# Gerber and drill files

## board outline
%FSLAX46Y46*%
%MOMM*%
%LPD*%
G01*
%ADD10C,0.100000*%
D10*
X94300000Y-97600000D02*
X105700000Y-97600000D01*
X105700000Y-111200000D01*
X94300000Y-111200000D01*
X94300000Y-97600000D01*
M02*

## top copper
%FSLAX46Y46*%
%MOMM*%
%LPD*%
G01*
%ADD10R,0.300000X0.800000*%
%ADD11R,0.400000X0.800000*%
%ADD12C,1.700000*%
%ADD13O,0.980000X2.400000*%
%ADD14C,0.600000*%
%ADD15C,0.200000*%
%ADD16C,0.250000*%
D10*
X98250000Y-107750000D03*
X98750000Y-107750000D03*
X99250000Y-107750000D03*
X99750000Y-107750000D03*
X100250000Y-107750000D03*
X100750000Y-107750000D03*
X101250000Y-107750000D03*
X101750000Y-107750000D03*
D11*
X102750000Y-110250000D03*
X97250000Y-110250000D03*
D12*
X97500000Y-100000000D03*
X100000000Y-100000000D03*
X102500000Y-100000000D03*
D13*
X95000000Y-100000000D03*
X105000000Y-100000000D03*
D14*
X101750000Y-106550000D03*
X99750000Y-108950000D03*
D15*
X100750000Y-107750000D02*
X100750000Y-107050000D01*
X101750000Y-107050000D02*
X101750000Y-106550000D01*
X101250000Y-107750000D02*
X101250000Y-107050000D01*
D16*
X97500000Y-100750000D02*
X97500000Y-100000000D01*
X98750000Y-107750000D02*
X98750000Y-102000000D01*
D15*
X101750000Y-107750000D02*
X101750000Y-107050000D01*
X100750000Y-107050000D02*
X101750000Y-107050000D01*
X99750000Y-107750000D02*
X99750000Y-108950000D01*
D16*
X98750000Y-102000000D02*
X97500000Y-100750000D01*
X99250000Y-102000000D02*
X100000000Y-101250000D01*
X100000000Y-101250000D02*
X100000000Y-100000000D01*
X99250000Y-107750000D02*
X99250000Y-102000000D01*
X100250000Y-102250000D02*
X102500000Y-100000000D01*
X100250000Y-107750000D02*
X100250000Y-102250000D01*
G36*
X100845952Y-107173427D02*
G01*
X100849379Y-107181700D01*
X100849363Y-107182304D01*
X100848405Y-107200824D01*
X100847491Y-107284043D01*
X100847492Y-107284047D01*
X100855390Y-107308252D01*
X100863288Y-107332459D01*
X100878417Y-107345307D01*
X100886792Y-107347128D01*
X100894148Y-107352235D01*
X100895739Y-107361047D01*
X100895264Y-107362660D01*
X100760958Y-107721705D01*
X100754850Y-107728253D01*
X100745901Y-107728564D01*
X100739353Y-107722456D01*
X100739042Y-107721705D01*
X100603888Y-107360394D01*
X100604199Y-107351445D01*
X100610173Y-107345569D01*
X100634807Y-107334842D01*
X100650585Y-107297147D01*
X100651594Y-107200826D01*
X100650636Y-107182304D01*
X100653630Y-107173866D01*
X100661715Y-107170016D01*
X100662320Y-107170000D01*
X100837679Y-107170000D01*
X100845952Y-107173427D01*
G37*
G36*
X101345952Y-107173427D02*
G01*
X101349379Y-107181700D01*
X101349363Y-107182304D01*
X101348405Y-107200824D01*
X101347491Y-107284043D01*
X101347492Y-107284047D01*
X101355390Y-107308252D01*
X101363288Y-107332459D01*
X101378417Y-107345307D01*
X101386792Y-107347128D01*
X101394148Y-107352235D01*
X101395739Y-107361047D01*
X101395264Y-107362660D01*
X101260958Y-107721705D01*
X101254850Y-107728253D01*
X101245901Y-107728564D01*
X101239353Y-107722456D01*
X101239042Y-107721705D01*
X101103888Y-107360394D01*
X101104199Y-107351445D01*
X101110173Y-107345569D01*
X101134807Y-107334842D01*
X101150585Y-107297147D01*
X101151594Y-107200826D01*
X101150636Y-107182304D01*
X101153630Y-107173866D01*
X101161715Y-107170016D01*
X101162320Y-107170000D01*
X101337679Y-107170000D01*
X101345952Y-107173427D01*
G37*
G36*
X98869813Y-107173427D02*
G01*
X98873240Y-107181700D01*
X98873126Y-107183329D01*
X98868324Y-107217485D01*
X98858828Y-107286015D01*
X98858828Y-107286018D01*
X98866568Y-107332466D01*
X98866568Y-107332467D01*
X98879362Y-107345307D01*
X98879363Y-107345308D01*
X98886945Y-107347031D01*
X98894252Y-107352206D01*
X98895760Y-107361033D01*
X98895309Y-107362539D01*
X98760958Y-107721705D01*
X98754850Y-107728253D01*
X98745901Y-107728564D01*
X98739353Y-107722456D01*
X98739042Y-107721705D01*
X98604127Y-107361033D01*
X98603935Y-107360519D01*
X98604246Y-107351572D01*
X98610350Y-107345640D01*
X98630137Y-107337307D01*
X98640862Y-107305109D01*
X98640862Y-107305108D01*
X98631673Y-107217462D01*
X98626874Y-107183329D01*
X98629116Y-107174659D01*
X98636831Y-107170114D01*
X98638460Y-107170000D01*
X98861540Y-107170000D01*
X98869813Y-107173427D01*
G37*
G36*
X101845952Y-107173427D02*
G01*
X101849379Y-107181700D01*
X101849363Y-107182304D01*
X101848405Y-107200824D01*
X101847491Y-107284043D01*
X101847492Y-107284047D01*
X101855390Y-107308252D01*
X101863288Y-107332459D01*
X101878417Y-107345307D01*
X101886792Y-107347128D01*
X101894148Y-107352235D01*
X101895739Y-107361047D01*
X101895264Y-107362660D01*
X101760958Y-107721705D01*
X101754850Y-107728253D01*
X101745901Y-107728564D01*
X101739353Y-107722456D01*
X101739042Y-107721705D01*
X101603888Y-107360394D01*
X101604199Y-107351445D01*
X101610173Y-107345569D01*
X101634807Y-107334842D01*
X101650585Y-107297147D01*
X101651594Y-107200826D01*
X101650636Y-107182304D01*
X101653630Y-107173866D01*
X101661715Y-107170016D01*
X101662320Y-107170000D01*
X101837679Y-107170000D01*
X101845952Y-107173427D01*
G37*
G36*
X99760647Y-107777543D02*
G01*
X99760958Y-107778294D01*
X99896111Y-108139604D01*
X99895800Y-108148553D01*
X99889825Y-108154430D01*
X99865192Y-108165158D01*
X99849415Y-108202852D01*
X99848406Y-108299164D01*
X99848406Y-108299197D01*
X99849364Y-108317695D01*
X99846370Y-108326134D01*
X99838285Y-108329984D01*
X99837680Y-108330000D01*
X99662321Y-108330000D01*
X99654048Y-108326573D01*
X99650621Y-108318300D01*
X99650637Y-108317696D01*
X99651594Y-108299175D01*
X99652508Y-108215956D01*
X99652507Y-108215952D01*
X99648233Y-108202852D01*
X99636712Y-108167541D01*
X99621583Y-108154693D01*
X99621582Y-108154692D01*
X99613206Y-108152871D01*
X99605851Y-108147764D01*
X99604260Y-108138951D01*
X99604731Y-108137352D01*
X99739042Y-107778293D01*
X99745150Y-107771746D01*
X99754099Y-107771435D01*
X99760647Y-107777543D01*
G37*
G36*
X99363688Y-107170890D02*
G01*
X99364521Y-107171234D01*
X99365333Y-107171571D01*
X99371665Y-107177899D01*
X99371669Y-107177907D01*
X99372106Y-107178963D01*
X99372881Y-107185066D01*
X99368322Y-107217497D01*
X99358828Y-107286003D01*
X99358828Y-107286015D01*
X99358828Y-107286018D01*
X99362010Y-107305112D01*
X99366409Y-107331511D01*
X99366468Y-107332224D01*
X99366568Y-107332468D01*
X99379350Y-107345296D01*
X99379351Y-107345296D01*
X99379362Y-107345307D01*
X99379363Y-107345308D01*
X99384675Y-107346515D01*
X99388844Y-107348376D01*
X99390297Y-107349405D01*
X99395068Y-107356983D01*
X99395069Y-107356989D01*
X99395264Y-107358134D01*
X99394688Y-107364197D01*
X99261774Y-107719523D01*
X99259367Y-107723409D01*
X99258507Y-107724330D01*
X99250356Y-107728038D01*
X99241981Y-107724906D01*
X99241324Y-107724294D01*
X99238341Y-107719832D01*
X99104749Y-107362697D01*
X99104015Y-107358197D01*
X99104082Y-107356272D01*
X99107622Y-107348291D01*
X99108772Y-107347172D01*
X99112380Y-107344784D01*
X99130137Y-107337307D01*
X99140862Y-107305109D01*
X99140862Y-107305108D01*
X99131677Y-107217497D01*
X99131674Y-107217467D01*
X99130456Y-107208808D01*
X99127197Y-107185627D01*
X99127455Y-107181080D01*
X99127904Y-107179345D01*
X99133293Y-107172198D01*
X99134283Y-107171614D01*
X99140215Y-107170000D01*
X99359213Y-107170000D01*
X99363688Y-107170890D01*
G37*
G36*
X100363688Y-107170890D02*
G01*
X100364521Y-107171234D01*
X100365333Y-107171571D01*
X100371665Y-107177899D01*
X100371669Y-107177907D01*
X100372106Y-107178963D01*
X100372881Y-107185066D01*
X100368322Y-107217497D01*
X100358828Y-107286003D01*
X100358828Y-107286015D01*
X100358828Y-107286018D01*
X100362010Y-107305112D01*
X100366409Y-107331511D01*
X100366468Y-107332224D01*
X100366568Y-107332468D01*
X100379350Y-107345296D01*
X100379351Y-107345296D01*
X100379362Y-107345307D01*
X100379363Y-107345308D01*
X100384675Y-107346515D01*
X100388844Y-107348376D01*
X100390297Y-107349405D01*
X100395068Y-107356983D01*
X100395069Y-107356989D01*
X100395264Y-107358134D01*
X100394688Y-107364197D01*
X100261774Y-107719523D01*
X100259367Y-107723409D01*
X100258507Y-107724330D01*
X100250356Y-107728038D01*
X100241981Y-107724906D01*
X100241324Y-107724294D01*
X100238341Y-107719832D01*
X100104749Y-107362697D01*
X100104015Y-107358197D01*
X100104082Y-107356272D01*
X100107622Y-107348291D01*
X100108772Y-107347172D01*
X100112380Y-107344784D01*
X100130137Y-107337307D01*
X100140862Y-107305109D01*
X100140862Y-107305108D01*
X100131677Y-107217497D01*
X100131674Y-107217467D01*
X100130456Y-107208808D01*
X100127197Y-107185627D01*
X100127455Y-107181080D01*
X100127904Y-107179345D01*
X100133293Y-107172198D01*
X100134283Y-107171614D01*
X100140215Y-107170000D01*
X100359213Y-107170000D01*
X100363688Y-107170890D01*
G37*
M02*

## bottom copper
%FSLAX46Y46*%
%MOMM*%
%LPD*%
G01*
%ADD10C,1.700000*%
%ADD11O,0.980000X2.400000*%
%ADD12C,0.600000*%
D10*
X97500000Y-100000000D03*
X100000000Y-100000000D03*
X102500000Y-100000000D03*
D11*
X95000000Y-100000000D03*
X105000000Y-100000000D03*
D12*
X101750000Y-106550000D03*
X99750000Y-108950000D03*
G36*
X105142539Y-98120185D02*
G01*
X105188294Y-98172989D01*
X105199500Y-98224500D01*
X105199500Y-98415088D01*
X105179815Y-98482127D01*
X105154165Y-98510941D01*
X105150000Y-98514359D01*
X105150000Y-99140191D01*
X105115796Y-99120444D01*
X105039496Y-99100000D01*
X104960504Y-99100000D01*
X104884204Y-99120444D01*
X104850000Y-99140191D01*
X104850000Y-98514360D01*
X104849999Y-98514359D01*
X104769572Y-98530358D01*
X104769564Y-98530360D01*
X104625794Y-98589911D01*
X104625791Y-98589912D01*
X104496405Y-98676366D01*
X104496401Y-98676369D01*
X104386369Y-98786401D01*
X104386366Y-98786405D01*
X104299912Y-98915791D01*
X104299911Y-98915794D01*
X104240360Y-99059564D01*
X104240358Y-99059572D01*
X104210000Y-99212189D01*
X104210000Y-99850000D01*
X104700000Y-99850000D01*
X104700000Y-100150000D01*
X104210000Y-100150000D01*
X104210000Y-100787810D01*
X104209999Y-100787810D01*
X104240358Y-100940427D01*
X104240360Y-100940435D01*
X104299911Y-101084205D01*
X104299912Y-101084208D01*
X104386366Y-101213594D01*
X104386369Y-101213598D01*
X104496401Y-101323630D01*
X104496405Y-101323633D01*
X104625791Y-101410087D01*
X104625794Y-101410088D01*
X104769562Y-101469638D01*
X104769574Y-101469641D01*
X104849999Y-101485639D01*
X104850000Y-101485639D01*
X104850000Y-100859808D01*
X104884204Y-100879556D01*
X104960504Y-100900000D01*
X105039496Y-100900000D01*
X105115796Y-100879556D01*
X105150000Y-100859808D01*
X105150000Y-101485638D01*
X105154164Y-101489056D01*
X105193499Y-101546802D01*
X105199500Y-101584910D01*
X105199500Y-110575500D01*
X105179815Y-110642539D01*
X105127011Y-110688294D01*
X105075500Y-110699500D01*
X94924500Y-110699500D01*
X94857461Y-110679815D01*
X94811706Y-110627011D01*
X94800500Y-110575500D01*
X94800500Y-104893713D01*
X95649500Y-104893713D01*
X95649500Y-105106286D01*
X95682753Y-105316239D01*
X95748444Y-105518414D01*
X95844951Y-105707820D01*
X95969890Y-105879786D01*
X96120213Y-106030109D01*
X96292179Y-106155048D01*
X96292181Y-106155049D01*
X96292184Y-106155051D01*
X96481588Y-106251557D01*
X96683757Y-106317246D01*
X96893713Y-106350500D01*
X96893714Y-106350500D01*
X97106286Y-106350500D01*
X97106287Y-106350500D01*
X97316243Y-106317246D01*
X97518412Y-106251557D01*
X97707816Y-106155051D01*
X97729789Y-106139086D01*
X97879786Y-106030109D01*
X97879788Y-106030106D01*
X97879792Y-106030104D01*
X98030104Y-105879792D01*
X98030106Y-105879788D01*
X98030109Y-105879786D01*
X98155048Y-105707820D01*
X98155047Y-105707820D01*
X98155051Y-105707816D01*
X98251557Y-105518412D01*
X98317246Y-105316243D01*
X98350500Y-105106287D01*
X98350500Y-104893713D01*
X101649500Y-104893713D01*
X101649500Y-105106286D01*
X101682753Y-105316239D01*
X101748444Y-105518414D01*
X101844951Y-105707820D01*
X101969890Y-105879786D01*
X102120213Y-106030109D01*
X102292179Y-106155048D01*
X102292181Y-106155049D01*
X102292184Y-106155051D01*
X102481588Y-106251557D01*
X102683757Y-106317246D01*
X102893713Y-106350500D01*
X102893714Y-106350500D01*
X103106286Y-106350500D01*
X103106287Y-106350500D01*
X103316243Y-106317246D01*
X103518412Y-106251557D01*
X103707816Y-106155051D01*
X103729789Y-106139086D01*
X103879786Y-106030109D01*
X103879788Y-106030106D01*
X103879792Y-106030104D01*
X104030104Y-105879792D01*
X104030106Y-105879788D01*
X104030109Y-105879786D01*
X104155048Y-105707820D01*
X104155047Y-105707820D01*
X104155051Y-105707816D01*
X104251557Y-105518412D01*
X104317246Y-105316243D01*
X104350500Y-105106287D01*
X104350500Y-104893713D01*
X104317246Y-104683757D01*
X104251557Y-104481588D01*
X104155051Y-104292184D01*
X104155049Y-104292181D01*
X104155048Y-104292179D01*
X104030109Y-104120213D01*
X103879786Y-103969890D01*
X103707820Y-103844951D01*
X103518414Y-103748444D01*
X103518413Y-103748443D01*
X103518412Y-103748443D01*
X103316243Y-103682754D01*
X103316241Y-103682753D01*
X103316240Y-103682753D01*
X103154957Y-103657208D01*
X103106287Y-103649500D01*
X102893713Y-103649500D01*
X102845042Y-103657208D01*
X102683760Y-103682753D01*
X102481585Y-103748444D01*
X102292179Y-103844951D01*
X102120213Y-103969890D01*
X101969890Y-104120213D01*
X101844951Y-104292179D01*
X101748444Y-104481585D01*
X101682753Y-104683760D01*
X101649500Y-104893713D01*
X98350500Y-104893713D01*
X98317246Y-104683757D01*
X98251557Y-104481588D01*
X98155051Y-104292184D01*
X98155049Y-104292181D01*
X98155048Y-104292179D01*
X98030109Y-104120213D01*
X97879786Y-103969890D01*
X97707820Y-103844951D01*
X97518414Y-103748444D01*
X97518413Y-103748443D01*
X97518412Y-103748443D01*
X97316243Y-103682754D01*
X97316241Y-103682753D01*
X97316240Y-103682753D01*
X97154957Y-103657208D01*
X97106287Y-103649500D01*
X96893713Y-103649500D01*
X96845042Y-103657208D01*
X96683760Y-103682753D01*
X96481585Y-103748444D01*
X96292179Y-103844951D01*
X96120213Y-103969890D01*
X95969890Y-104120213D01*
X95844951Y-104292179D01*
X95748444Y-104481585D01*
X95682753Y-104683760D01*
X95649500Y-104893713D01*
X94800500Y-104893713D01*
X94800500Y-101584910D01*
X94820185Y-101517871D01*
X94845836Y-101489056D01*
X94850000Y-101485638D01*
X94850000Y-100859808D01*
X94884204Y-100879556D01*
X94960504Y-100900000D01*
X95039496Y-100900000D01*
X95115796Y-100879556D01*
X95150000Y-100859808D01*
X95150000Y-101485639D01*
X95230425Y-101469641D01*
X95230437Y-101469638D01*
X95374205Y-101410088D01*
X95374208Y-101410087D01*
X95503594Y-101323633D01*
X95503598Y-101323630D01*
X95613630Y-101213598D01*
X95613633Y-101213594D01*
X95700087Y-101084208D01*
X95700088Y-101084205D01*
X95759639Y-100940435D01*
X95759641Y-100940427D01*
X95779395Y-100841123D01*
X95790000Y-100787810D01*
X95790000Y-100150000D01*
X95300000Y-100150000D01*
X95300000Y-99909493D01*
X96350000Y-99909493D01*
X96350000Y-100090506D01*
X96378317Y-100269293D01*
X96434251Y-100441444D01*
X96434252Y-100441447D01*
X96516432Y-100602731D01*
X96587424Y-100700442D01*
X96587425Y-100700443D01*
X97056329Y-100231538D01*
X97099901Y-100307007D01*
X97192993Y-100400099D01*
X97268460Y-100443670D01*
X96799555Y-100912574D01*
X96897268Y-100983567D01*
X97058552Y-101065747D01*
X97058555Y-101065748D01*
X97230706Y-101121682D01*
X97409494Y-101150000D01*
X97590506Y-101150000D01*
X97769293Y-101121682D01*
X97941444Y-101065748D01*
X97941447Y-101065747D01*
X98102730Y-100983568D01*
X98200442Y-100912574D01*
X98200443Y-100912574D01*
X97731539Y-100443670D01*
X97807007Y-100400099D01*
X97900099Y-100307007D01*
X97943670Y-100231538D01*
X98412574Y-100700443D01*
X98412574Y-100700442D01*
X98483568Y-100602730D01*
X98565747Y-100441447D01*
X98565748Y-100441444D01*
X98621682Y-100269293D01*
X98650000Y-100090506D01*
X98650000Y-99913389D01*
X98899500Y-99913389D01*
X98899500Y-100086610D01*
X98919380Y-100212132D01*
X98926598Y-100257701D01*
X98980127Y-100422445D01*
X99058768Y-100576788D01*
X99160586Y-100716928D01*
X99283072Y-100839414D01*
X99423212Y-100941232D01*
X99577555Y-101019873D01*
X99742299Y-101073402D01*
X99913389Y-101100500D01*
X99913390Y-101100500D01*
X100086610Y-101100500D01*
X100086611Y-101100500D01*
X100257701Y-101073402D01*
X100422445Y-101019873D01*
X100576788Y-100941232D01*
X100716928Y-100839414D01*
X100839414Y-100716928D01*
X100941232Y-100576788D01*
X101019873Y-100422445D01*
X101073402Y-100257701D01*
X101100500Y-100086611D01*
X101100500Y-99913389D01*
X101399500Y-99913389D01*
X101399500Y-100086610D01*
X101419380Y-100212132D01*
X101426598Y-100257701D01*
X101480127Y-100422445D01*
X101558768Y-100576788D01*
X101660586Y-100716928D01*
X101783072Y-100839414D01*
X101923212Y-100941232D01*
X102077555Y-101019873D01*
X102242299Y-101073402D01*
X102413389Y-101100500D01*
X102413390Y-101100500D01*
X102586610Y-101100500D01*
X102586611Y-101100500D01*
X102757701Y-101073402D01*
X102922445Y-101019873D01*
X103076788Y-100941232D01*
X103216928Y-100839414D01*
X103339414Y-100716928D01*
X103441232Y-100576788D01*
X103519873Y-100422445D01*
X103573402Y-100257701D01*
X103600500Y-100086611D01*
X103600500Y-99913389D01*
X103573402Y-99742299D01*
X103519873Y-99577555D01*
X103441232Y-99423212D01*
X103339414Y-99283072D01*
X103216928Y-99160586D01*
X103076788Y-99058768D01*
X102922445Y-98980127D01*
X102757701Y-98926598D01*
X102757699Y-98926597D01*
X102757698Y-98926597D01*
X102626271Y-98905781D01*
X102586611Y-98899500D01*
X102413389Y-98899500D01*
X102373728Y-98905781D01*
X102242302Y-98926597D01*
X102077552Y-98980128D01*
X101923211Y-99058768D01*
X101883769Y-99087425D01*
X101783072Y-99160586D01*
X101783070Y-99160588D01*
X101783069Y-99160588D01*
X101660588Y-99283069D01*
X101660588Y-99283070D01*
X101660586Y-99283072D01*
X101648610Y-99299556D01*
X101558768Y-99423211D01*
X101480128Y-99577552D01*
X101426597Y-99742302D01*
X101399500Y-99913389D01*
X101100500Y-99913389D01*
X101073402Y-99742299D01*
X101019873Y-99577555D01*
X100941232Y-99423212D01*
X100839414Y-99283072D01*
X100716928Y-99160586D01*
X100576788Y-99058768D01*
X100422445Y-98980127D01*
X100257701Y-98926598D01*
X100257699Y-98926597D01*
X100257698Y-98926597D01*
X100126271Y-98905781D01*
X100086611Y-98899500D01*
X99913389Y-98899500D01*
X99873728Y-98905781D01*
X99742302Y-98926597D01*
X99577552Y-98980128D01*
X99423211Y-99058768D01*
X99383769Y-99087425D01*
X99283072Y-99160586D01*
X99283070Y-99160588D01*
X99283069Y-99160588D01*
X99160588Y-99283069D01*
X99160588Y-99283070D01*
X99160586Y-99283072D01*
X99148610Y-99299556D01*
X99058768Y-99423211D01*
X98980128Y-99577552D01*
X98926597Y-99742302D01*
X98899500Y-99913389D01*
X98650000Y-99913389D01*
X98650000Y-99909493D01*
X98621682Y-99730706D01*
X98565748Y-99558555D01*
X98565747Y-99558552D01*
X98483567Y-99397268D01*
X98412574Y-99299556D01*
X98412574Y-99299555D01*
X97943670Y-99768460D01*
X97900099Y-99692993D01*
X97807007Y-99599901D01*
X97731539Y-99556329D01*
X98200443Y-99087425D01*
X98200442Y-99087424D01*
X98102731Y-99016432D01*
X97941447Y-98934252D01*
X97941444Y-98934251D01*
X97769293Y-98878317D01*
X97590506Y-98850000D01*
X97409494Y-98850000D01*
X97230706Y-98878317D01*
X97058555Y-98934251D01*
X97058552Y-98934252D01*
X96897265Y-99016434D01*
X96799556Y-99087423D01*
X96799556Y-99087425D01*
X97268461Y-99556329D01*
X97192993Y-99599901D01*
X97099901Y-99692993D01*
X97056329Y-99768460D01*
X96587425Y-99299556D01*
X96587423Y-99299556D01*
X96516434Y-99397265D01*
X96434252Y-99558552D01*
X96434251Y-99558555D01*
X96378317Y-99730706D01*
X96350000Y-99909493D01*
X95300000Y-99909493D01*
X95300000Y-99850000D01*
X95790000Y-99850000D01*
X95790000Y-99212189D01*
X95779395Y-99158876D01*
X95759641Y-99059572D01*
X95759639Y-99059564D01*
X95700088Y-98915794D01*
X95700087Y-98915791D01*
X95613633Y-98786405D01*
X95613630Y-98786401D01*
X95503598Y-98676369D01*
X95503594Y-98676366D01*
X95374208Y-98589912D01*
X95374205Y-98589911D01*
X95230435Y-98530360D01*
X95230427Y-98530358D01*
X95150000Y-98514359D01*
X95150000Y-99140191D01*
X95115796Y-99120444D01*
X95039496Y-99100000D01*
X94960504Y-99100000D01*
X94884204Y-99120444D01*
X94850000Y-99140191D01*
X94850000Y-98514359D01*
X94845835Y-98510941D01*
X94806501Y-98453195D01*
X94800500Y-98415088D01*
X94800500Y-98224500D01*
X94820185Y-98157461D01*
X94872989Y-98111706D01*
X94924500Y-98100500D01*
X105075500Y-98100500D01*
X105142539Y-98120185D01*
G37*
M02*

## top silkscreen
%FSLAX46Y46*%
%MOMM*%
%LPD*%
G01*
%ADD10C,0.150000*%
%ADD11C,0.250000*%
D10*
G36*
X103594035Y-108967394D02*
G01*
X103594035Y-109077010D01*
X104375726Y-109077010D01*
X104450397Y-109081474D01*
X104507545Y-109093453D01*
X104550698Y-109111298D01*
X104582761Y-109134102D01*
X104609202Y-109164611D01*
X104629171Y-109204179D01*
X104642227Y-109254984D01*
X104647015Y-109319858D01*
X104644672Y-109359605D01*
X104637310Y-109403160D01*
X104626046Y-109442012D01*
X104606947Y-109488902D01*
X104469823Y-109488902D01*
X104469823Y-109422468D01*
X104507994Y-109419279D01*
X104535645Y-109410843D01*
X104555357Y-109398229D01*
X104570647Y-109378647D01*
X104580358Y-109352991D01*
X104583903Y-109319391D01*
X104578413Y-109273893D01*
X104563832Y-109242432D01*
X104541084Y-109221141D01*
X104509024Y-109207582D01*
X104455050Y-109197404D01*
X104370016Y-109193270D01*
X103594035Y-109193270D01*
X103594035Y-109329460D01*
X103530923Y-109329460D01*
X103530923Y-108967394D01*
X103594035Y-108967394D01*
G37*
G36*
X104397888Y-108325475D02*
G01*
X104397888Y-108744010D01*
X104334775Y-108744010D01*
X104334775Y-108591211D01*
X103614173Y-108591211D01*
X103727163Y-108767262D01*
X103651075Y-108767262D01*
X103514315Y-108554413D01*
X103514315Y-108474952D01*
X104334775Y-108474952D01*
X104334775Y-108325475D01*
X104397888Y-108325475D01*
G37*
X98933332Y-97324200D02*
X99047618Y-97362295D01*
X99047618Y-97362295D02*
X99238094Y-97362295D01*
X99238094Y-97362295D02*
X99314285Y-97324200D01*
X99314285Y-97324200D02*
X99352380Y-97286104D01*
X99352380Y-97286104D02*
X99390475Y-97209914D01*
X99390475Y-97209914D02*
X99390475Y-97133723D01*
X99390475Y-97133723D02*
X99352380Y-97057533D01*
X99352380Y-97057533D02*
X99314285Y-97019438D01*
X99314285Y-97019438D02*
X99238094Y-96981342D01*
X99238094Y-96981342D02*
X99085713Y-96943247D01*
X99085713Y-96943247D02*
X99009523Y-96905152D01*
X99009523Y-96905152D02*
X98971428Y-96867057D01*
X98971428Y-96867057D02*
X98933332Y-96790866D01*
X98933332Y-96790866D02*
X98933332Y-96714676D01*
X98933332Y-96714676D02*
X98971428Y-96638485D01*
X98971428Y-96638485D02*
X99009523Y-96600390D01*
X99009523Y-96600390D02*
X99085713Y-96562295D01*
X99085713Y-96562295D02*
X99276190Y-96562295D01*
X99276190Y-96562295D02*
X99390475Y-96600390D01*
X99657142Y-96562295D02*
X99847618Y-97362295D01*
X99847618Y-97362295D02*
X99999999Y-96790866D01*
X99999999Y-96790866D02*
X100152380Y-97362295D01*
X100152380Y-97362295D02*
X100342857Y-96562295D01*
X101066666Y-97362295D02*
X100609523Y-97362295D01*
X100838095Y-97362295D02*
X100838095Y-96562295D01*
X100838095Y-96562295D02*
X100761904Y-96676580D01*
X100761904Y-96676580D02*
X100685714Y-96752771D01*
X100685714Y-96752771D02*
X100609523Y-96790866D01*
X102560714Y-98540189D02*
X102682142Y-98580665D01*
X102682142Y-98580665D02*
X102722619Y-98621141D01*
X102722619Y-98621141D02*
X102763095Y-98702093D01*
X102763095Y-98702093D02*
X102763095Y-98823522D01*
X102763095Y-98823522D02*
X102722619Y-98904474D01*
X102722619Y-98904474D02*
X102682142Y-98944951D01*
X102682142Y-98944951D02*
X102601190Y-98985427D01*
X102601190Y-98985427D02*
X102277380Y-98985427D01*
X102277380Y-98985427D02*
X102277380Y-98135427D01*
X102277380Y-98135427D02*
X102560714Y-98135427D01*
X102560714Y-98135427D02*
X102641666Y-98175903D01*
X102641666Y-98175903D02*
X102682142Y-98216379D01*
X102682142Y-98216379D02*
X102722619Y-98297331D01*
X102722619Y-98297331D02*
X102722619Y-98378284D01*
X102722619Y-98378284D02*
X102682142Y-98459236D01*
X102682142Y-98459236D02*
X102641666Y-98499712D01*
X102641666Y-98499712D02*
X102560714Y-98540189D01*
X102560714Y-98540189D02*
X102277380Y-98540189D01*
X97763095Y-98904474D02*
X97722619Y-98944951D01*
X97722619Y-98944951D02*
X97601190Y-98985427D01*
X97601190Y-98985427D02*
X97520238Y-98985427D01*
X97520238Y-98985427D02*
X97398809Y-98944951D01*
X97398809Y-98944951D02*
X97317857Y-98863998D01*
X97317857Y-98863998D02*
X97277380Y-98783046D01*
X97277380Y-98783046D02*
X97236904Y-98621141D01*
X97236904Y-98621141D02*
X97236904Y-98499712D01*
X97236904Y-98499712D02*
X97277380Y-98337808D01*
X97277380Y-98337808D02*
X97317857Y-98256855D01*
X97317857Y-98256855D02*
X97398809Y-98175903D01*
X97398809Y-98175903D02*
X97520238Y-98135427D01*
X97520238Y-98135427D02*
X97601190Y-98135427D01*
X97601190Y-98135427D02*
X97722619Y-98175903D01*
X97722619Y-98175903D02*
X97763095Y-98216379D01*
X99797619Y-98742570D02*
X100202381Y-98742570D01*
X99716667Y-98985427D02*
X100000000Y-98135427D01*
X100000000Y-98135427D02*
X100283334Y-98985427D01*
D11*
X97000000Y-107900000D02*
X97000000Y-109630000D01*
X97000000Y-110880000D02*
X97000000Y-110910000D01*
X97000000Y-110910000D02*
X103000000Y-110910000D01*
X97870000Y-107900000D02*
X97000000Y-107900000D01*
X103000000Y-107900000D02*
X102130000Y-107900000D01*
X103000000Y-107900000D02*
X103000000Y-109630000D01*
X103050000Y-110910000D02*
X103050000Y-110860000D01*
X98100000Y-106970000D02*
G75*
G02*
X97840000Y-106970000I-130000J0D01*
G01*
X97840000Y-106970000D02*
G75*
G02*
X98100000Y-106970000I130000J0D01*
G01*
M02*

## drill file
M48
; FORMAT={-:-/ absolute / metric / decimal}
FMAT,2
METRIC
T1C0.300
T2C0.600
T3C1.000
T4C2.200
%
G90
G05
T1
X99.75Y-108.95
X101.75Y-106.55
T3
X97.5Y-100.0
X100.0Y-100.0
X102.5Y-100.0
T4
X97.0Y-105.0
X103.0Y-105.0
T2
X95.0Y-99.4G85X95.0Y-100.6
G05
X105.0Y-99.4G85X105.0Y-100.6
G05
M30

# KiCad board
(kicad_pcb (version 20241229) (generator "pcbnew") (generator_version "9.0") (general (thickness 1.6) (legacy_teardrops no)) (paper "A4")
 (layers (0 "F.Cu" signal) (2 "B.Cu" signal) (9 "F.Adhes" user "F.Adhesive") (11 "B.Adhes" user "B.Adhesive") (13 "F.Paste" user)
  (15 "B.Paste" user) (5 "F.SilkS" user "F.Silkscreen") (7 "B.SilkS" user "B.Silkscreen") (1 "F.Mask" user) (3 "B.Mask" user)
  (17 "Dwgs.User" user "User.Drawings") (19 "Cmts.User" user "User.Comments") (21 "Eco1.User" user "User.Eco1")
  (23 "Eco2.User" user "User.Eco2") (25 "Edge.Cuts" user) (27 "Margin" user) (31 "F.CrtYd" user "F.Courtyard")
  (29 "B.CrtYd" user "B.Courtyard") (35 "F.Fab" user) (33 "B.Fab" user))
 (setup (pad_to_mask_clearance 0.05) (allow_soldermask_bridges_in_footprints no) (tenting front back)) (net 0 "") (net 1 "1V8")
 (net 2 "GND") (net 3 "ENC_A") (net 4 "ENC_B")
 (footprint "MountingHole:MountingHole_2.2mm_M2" (layer "F.Cu") (at 103 105)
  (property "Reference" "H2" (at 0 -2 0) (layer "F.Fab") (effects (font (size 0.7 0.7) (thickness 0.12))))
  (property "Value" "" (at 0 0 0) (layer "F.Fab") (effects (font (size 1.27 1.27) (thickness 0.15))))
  (pad "" np_thru_hole circle (at 0 0) (size 2.2 2.2) (drill 2.2) (layers "*.Cu" "*.Mask")))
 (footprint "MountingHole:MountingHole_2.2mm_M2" (layer "F.Cu") (at 97 105)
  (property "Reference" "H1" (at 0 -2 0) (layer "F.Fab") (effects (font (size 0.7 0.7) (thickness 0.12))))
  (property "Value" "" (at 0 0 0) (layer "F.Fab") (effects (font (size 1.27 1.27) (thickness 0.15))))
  (pad "" np_thru_hole circle (at 0 0) (size 2.2 2.2) (drill 2.2) (layers "*.Cu" "*.Mask")))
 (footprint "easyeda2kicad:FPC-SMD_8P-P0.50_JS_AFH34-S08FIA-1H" (layer "F.Cu") (at 100 109 180)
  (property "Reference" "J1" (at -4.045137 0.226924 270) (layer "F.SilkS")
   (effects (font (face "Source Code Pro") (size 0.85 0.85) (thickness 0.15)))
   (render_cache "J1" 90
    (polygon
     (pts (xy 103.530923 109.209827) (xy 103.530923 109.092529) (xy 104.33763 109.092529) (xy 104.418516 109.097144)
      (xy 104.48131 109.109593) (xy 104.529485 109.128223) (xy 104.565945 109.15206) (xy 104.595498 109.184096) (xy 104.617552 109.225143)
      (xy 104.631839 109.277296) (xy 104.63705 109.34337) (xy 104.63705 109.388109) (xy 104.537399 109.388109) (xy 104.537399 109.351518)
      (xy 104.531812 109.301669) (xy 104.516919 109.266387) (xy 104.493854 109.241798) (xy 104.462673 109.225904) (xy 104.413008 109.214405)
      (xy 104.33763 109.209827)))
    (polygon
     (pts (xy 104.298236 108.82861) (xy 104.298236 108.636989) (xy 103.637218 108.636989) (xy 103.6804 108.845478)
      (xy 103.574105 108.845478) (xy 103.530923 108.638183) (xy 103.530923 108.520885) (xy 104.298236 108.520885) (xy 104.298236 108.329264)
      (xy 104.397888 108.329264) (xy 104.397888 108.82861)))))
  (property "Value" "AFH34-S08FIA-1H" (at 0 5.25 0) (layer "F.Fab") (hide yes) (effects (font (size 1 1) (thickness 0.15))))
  (fp_line (start 3 1.1) (end 3 -0.63) (stroke (width 0.25) (type solid)) (layer "F.SilkS"))
  (fp_line (start 3 -1.88) (end 3 -1.91) (stroke (width 0.25) (type solid)) (layer "F.SilkS"))
  (fp_line (start 3 -1.91) (end -3 -1.91) (stroke (width 0.25) (type solid)) (layer "F.SilkS"))
  (fp_line (start 2.13 1.1) (end 3 1.1) (stroke (width 0.25) (type solid)) (layer "F.SilkS"))
  (fp_line (start -3 1.1) (end -2.13 1.1) (stroke (width 0.25) (type solid)) (layer "F.SilkS"))
  (fp_line (start -3 1.1) (end -3 -0.63) (stroke (width 0.25) (type solid)) (layer "F.SilkS"))
  (fp_line (start -3.05 -1.91) (end -3.05 -1.86) (stroke (width 0.25) (type solid)) (layer "F.SilkS"))
  (fp_circle (center 2.03 2.03) (end 2.16 2.03) (stroke (width 0.25) (type solid)) (fill no) (layer "F.SilkS"))
  (pad "1" smd rect (at 1.75 1.25) (size 0.3 0.8) (layers "F.Cu" "F.Mask" "F.Paste") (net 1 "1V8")
   (teardrops (best_length_ratio 0.6) (max_length 0.35) (best_width_ratio 1) (max_width 2) (curved_edges yes) (filter_ratio 0.9)
    (enabled yes) (allow_two_segments yes) (prefer_zone_connections yes)))
  (pad "2" smd rect (at 1.25 1.25) (size 0.3 0.8) (layers "F.Cu" "F.Mask" "F.Paste") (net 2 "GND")
   (teardrops (best_length_ratio 0.6) (max_length 0.35) (best_width_ratio 1) (max_width 2) (curved_edges yes) (filter_ratio 0.9)
    (enabled yes) (allow_two_segments yes) (prefer_zone_connections yes)))
  (pad "3" smd rect (at 0.75 1.25) (size 0.3 0.8) (layers "F.Cu" "F.Mask" "F.Paste") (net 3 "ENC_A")
   (teardrops (best_length_ratio 0.6) (max_length 0.35) (best_width_ratio 1) (max_width 2) (curved_edges yes) (filter_ratio 0.9)
    (enabled yes) (allow_two_segments yes) (prefer_zone_connections yes)))
  (pad "4" smd rect (at 0.25 1.25) (size 0.3 0.8) (layers "F.Cu" "F.Mask" "F.Paste") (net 2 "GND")
   (teardrops (best_length_ratio 0.6) (max_length 0.35) (best_width_ratio 1) (max_width 2) (curved_edges yes) (filter_ratio 0.9)
    (enabled yes) (allow_two_segments yes) (prefer_zone_connections yes)))
  (pad "5" smd rect (at -0.25 1.25) (size 0.3 0.8) (layers "F.Cu" "F.Mask" "F.Paste") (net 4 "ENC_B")
   (teardrops (best_length_ratio 0.6) (max_length 0.35) (best_width_ratio 1) (max_width 2) (curved_edges yes) (filter_ratio 0.9)
    (enabled yes) (allow_two_segments yes) (prefer_zone_connections yes)))
  (pad "6" smd rect (at -0.75 1.25) (size 0.3 0.8) (layers "F.Cu" "F.Mask" "F.Paste") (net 2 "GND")
   (teardrops (best_length_ratio 0.6) (max_length 0.35) (best_width_ratio 1) (max_width 2) (curved_edges yes) (filter_ratio 0.9)
    (enabled yes) (allow_two_segments yes) (prefer_zone_connections yes)))
  (pad "7" smd rect (at -1.25 1.25) (size 0.3 0.8) (layers "F.Cu" "F.Mask" "F.Paste") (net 2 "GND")
   (teardrops (best_length_ratio 0.6) (max_length 0.35) (best_width_ratio 1) (max_width 2) (curved_edges yes) (filter_ratio 0.9)
    (enabled yes) (allow_two_segments yes) (prefer_zone_connections yes)))
  (pad "8" smd rect (at -1.75 1.25) (size 0.3 0.8) (layers "F.Cu" "F.Mask" "F.Paste") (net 2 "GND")
   (teardrops (best_length_ratio 0.6) (max_length 0.35) (best_width_ratio 1) (max_width 2) (curved_edges yes) (filter_ratio 0.9)
    (enabled yes) (allow_two_segments yes) (prefer_zone_connections yes)))
  (pad "9" smd rect (at -2.75 -1.25) (size 0.4 0.8) (layers "F.Cu" "F.Mask" "F.Paste")
   (teardrops (best_length_ratio 0.6) (max_length 0.35) (best_width_ratio 1) (max_width 2) (curved_edges yes) (filter_ratio 0.9)
    (enabled yes) (allow_two_segments yes) (prefer_zone_connections yes)))
  (pad "10" smd rect (at 2.75 -1.25) (size 0.4 0.8) (layers "F.Cu" "F.Mask" "F.Paste")
   (teardrops (best_length_ratio 0.6) (max_length 0.35) (best_width_ratio 1) (max_width 2) (curved_edges yes) (filter_ratio 0.9)
    (enabled yes) (allow_two_segments yes) (prefer_zone_connections yes))))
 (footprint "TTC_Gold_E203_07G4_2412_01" (layer "F.Cu") (at 100 100)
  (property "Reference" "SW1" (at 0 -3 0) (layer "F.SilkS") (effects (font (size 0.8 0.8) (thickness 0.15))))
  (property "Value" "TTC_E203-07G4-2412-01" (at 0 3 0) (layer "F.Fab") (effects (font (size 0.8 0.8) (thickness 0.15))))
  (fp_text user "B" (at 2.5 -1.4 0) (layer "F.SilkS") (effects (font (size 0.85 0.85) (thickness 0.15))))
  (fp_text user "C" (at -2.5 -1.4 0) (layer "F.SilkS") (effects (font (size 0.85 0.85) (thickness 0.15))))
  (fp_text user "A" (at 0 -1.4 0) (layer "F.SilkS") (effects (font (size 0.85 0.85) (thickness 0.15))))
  (pad "1" thru_hole circle (at -2.5 0) (size 1.7 1.7) (drill 1) (layers "*.Cu" "*.Mask") (remove_unused_layers no) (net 2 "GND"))
  (pad "2" thru_hole circle (at 0 0) (size 1.7 1.7) (drill 1) (layers "*.Cu" "*.Mask") (remove_unused_layers no) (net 3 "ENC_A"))
  (pad "3" thru_hole circle (at 2.5 0) (size 1.7 1.7) (drill 1) (layers "*.Cu" "*.Mask") (remove_unused_layers no) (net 4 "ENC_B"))
  (pad "MP1" thru_hole oval (at -5 0) (size 0.98 2.4) (drill oval 0.6 1.8) (layers "*.Cu" "*.Mask") (remove_unused_layers no) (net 2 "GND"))
  (pad "MP2" thru_hole oval (at 5 0) (size 0.98 2.4) (drill oval 0.6 1.8) (layers "*.Cu" "*.Mask") (remove_unused_layers no) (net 2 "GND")))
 (gr_rect (start 94.3 97.6) (end 105.7 111.2) (stroke (width 0.1) (type solid)) (fill no) (layer "Edge.Cuts"))
 (segment (start 100.75 107.75) (end 100.75 107.05) (width 0.2) (layer "F.Cu") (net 2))
 (segment (start 101.75 107.05) (end 101.75 106.55) (width 0.2) (layer "F.Cu") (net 2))
 (segment (start 101.25 107.75) (end 101.25 107.05) (width 0.2) (layer "F.Cu") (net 2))
 (segment (start 97.5 100.75) (end 97.5 100) (width 0.25) (layer "F.Cu") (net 2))
 (segment (start 98.75 107.75) (end 98.75 102) (width 0.25) (layer "F.Cu") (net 2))
 (segment (start 101.75 107.75) (end 101.75 107.05) (width 0.2) (layer "F.Cu") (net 2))
 (segment (start 100.75 107.05) (end 101.75 107.05) (width 0.2) (layer "F.Cu") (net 2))
 (segment (start 99.75 107.75) (end 99.75 108.95) (width 0.2) (layer "F.Cu") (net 2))
 (segment (start 98.75 102) (end 97.5 100.75) (width 0.25) (layer "F.Cu") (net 2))
 (via (at 101.75 106.55) (size 0.6) (drill 0.3) (layers "F.Cu" "B.Cu") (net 2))
 (via (at 99.75 108.95) (size 0.6) (drill 0.3) (layers "F.Cu" "B.Cu") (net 2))
 (segment (start 99.25 102) (end 100 101.25) (width 0.25) (layer "F.Cu") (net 3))
 (segment (start 100 101.25) (end 100 100) (width 0.25) (layer "F.Cu") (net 3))
 (segment (start 99.25 107.75) (end 99.25 102) (width 0.25) (layer "F.Cu") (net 3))
 (segment (start 100.25 102.25) (end 102.5 100) (width 0.25) (layer "F.Cu") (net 4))
 (segment (start 100.25 107.75) (end 100.25 102.25) (width 0.25) (layer "F.Cu") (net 4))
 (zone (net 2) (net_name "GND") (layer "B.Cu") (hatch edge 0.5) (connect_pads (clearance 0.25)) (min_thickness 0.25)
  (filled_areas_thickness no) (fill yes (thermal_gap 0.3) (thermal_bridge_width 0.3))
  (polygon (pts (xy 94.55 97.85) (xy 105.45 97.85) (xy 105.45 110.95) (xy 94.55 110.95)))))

